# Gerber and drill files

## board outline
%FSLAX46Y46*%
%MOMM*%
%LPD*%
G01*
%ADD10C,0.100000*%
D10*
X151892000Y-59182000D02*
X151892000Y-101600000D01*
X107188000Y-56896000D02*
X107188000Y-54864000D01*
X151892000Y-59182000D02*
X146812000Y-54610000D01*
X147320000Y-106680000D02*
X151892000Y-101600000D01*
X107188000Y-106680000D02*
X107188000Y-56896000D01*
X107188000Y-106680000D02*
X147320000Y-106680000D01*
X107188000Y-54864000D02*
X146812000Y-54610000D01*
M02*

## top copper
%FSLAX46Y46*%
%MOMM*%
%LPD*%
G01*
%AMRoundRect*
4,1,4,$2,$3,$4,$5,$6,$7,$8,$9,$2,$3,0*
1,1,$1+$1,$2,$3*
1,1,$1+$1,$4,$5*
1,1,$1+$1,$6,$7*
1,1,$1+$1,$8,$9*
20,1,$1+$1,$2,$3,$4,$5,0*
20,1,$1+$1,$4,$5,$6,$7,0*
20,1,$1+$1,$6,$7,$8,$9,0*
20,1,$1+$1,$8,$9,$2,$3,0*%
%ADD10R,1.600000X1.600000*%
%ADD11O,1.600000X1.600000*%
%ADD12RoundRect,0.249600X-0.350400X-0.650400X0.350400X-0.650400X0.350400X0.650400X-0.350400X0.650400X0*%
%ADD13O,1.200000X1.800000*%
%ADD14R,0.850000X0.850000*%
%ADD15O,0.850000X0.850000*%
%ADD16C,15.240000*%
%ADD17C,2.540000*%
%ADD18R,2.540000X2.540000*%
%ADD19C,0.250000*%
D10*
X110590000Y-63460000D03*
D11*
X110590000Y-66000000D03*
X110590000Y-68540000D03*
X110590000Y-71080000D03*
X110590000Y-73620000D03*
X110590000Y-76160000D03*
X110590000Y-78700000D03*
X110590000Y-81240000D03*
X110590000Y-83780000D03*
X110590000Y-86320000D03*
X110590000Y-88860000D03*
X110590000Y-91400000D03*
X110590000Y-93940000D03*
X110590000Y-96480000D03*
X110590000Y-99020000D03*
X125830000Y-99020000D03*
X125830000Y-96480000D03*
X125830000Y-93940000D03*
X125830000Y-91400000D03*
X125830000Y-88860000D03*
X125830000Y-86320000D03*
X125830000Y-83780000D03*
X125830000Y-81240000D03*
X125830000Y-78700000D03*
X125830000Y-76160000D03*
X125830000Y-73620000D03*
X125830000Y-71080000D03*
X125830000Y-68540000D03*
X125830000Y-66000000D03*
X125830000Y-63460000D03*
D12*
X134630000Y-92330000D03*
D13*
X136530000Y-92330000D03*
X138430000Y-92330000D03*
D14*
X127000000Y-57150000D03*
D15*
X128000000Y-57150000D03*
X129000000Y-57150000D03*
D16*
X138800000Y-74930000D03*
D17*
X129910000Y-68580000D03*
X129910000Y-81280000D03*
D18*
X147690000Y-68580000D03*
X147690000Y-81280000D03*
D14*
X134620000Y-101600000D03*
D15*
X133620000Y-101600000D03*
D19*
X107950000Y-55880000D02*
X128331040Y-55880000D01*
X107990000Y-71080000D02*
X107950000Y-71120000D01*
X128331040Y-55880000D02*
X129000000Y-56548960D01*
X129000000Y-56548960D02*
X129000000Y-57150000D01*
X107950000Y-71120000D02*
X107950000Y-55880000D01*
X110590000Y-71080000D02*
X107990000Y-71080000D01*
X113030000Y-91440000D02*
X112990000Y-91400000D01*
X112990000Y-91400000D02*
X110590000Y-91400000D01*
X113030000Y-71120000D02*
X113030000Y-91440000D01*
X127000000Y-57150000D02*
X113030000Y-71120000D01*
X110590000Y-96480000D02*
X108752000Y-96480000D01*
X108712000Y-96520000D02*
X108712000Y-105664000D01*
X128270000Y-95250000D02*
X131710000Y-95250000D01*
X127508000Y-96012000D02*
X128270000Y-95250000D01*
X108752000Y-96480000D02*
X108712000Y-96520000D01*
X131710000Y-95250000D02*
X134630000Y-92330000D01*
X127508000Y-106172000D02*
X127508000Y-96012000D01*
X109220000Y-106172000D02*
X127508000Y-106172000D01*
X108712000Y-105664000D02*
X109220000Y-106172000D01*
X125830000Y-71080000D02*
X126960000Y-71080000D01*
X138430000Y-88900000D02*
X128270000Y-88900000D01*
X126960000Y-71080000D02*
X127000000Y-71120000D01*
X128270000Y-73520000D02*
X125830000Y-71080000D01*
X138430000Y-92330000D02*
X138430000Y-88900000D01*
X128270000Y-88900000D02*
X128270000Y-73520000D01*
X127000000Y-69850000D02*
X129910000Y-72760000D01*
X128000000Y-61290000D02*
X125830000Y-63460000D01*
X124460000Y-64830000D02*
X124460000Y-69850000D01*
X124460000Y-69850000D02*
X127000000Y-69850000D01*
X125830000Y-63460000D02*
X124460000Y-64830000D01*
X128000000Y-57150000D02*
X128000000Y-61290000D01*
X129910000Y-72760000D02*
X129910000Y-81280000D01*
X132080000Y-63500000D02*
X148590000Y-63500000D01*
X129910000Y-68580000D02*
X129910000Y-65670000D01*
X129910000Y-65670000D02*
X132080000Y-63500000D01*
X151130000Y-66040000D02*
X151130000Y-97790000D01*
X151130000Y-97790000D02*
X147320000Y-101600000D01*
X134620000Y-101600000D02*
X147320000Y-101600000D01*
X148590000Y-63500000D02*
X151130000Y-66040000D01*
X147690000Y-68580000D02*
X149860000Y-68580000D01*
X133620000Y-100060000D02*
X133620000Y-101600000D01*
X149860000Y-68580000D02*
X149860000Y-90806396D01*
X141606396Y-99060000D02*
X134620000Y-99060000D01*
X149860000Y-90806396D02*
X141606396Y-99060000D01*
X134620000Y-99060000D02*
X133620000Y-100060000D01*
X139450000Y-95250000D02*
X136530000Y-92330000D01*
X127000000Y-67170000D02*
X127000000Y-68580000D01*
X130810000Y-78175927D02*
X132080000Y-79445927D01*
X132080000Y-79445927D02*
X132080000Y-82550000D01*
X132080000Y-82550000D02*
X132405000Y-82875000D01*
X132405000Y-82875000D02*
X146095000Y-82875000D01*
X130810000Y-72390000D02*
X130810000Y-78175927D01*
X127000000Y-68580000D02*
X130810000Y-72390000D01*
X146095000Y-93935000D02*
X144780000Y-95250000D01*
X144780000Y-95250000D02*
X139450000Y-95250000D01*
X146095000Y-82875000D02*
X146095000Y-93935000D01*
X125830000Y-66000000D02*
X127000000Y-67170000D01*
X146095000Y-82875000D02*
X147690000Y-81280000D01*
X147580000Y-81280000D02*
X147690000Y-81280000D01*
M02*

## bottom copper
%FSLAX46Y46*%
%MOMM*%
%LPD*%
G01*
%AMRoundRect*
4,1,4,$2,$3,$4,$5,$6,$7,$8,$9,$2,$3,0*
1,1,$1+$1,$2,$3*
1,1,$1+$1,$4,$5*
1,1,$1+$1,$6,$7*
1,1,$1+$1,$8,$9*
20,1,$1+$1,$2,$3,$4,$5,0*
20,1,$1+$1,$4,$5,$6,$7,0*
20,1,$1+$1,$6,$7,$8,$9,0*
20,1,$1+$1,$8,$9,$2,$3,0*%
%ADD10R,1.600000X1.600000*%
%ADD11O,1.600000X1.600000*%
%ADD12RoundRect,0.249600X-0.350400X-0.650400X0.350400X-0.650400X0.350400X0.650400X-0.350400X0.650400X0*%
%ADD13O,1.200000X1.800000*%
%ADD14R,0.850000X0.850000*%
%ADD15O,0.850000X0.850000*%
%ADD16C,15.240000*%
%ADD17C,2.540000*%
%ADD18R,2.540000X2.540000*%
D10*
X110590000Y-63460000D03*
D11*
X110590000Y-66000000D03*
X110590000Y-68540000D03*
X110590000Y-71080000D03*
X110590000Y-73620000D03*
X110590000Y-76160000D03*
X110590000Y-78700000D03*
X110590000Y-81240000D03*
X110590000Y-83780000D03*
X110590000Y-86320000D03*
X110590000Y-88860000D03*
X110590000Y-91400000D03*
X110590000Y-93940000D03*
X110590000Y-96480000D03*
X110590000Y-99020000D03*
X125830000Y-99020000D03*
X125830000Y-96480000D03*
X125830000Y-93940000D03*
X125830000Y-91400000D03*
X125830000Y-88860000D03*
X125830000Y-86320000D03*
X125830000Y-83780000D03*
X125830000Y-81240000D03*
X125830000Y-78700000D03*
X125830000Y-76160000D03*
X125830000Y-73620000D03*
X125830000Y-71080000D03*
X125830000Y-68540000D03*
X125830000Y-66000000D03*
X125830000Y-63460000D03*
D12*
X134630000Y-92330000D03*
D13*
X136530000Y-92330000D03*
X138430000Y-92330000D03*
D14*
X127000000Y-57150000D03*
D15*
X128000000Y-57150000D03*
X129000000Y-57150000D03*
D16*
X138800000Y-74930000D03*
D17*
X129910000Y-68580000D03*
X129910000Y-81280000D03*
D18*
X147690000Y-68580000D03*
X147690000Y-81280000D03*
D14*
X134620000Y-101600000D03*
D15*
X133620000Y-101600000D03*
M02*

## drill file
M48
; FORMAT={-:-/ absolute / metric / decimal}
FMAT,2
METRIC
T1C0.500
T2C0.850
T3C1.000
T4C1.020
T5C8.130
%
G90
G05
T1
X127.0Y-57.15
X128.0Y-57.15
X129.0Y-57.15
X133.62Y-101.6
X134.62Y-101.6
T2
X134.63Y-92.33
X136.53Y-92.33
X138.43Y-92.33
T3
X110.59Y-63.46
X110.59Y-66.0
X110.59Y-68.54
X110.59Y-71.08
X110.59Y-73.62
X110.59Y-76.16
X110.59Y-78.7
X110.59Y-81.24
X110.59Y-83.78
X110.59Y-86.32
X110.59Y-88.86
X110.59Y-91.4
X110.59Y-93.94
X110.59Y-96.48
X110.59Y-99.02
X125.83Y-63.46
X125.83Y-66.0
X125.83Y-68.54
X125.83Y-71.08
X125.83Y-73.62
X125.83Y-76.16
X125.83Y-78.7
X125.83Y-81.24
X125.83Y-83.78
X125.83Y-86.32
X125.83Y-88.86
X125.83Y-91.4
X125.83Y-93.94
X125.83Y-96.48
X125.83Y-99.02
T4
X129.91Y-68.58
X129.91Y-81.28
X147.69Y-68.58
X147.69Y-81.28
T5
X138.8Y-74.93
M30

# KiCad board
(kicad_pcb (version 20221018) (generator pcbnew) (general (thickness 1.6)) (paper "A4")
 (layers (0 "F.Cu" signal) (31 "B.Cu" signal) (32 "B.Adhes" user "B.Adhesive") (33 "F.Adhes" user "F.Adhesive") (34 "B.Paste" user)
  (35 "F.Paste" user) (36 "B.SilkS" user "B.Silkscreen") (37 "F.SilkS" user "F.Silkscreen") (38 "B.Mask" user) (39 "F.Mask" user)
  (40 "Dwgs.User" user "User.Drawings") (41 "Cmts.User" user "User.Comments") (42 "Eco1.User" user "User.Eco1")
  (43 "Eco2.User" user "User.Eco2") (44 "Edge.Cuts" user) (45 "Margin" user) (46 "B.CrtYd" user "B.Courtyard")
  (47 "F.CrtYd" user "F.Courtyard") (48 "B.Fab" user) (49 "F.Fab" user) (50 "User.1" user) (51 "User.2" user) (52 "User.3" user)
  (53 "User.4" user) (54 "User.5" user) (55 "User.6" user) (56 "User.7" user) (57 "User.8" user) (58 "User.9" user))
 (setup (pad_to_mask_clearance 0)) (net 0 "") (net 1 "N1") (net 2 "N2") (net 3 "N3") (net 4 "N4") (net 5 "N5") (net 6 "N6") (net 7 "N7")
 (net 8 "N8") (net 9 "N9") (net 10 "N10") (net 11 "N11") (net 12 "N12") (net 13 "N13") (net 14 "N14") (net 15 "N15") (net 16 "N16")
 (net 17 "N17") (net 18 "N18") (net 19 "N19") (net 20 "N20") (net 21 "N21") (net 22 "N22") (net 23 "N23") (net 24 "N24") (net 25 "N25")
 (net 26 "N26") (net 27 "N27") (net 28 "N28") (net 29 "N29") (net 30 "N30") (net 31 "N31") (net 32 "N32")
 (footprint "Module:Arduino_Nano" (layer "F.Cu") (at 110.59 63.46)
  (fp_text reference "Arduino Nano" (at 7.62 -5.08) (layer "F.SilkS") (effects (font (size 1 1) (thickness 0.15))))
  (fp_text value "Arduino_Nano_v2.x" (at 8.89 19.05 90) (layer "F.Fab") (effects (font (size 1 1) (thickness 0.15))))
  (pad "1" thru_hole rect (at 0 0) (size 1.6 1.6) (drill 1) (layers "*.Cu" "*.Mask") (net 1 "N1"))
  (pad "2" thru_hole oval (at 0 2.54) (size 1.6 1.6) (drill 1) (layers "*.Cu" "*.Mask") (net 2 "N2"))
  (pad "3" thru_hole oval (at 0 5.08) (size 1.6 1.6) (drill 1) (layers "*.Cu" "*.Mask") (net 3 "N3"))
  (pad "4" thru_hole oval (at 0 7.62) (size 1.6 1.6) (drill 1) (layers "*.Cu" "*.Mask") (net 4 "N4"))
  (pad "5" thru_hole oval (at 0 10.16) (size 1.6 1.6) (drill 1) (layers "*.Cu" "*.Mask") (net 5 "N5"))
  (pad "6" thru_hole oval (at 0 12.7) (size 1.6 1.6) (drill 1) (layers "*.Cu" "*.Mask") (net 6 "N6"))
  (pad "7" thru_hole oval (at 0 15.24) (size 1.6 1.6) (drill 1) (layers "*.Cu" "*.Mask") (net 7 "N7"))
  (pad "8" thru_hole oval (at 0 17.78) (size 1.6 1.6) (drill 1) (layers "*.Cu" "*.Mask") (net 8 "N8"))
  (pad "9" thru_hole oval (at 0 20.32) (size 1.6 1.6) (drill 1) (layers "*.Cu" "*.Mask") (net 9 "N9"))
  (pad "10" thru_hole oval (at 0 22.86) (size 1.6 1.6) (drill 1) (layers "*.Cu" "*.Mask") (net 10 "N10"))
  (pad "11" thru_hole oval (at 0 25.4) (size 1.6 1.6) (drill 1) (layers "*.Cu" "*.Mask") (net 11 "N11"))
  (pad "12" thru_hole oval (at 0 27.94) (size 1.6 1.6) (drill 1) (layers "*.Cu" "*.Mask") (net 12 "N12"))
  (pad "13" thru_hole oval (at 0 30.48) (size 1.6 1.6) (drill 1) (layers "*.Cu" "*.Mask") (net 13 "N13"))
  (pad "14" thru_hole oval (at 0 33.02) (size 1.6 1.6) (drill 1) (layers "*.Cu" "*.Mask") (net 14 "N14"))
  (pad "15" thru_hole oval (at 0 35.56) (size 1.6 1.6) (drill 1) (layers "*.Cu" "*.Mask") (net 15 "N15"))
  (pad "16" thru_hole oval (at 15.24 35.56) (size 1.6 1.6) (drill 1) (layers "*.Cu" "*.Mask") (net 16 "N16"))
  (pad "17" thru_hole oval (at 15.24 33.02) (size 1.6 1.6) (drill 1) (layers "*.Cu" "*.Mask") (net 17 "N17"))
  (pad "18" thru_hole oval (at 15.24 30.48) (size 1.6 1.6) (drill 1) (layers "*.Cu" "*.Mask") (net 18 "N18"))
  (pad "19" thru_hole oval (at 15.24 27.94) (size 1.6 1.6) (drill 1) (layers "*.Cu" "*.Mask") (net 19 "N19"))
  (pad "20" thru_hole oval (at 15.24 25.4) (size 1.6 1.6) (drill 1) (layers "*.Cu" "*.Mask") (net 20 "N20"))
  (pad "21" thru_hole oval (at 15.24 22.86) (size 1.6 1.6) (drill 1) (layers "*.Cu" "*.Mask") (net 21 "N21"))
  (pad "22" thru_hole oval (at 15.24 20.32) (size 1.6 1.6) (drill 1) (layers "*.Cu" "*.Mask") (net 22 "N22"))
  (pad "23" thru_hole oval (at 15.24 17.78) (size 1.6 1.6) (drill 1) (layers "*.Cu" "*.Mask") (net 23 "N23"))
  (pad "24" thru_hole oval (at 15.24 15.24) (size 1.6 1.6) (drill 1) (layers "*.Cu" "*.Mask") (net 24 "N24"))
  (pad "25" thru_hole oval (at 15.24 12.7) (size 1.6 1.6) (drill 1) (layers "*.Cu" "*.Mask") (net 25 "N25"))
  (pad "26" thru_hole oval (at 15.24 10.16) (size 1.6 1.6) (drill 1) (layers "*.Cu" "*.Mask") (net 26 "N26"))
  (pad "27" thru_hole oval (at 15.24 7.62) (size 1.6 1.6) (drill 1) (layers "*.Cu" "*.Mask") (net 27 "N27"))
  (pad "28" thru_hole oval (at 15.24 5.08) (size 1.6 1.6) (drill 1) (layers "*.Cu" "*.Mask") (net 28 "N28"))
  (pad "29" thru_hole oval (at 15.24 2.54) (size 1.6 1.6) (drill 1) (layers "*.Cu" "*.Mask") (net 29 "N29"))
  (pad "30" thru_hole oval (at 15.24 0) (size 1.6 1.6) (drill 1) (layers "*.Cu" "*.Mask") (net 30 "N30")))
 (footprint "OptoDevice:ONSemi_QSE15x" (layer "F.Cu") (at 134.63 92.33)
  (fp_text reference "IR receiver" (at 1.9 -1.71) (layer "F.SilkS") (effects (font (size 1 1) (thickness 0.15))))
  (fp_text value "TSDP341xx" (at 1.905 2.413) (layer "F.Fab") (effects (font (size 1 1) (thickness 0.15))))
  (pad "1" thru_hole roundrect (at 0 0) (size 1.2 1.8) (drill 0.85) (layers "*.Cu" "*.Mask") (roundrect_rratio 0.208) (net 14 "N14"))
  (pad "2" thru_hole oval (at 1.9 0) (size 1.2 1.8) (drill 0.85) (layers "*.Cu" "*.Mask") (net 29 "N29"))
  (pad "3" thru_hole oval (at 3.8 0) (size 1.2 1.8) (drill 0.85) (layers "*.Cu" "*.Mask") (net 27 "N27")))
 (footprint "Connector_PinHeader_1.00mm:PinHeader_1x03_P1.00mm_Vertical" (layer "F.Cu") (at 127 57.15 90)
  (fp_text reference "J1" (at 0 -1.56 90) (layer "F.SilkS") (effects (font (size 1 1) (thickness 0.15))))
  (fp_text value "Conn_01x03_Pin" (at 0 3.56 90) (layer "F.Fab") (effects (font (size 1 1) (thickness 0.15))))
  (pad "1" thru_hole rect (at 0 0 90) (size 0.85 0.85) (drill 0.5) (layers "*.Cu" "*.Mask") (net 12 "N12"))
  (pad "2" thru_hole oval (at 0 1 90) (size 0.85 0.85) (drill 0.5) (layers "*.Cu" "*.Mask") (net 30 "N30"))
  (pad "3" thru_hole oval (at 0 2 90) (size 0.85 0.85) (drill 0.5) (layers "*.Cu" "*.Mask") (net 4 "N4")))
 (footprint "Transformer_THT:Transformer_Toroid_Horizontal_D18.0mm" (layer "F.Cu") (at 129.91 68.58)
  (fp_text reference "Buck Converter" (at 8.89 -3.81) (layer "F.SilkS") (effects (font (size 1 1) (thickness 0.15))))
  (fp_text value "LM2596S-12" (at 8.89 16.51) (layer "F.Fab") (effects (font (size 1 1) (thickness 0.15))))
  (pad "" thru_hole circle (at 8.89 6.35) (size 15.24 15.24) (drill 8.13) (layers "*.Cu" "*.Mask"))
  (pad "1" thru_hole circle (at 0 0) (size 2.54 2.54) (drill 1.02) (layers "*.Cu" "*.Mask") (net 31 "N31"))
  (pad "2" thru_hole circle (at 0 12.7) (size 2.54 2.54) (drill 1.02) (layers "*.Cu" "*.Mask") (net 30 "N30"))
  (pad "3" thru_hole rect (at 17.78 0) (size 2.54 2.54) (drill 1.02) (layers "*.Cu" "*.Mask") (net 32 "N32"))
  (pad "4" thru_hole rect (at 17.78 12.7) (size 2.54 2.54) (drill 1.02) (layers "*.Cu" "*.Mask") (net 29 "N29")))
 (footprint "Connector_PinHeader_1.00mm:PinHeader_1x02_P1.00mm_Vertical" (layer "F.Cu") (at 134.62 101.6 -90)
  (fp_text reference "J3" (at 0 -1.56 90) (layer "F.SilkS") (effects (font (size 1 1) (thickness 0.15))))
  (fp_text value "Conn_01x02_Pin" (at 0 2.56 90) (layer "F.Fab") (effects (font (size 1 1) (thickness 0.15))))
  (pad "1" thru_hole rect (at 0 0 270) (size 0.85 0.85) (drill 0.5) (layers "*.Cu" "*.Mask") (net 31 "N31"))
  (pad "2" thru_hole oval (at 0 1 270) (size 0.85 0.85) (drill 0.5) (layers "*.Cu" "*.Mask") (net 32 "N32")))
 (gr_line (start 151.892 59.182) (end 151.892 101.6) (stroke (width 0.1) (type default)) (layer "Edge.Cuts"))
 (gr_line (start 107.188 56.896) (end 107.188 54.864) (stroke (width 0.1) (type default)) (layer "Edge.Cuts"))
 (gr_line (start 151.892 59.182) (end 146.812 54.61) (stroke (width 0.1) (type default)) (layer "Edge.Cuts"))
 (gr_line (start 147.32 106.68) (end 151.892 101.6) (stroke (width 0.1) (type default)) (layer "Edge.Cuts"))
 (gr_line (start 107.188 106.68) (end 107.188 56.896) (stroke (width 0.1) (type default)) (layer "Edge.Cuts"))
 (gr_line (start 107.188 106.68) (end 147.32 106.68) (stroke (width 0.1) (type default)) (layer "Edge.Cuts"))
 (gr_line (start 107.188 54.864) (end 146.812 54.61) (stroke (width 0.1) (type default)) (layer "Edge.Cuts"))
 (segment (start 107.95 55.88) (end 128.33104 55.88) (width 0.25) (layer "F.Cu") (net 4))
 (segment (start 107.99 71.08) (end 107.95 71.12) (width 0.25) (layer "F.Cu") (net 4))
 (segment (start 128.33104 55.88) (end 129 56.54896) (width 0.25) (layer "F.Cu") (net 4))
 (segment (start 129 56.54896) (end 129 57.15) (width 0.25) (layer "F.Cu") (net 4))
 (segment (start 107.95 71.12) (end 107.95 55.88) (width 0.25) (layer "F.Cu") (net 4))
 (segment (start 110.59 71.08) (end 107.99 71.08) (width 0.25) (layer "F.Cu") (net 4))
 (segment (start 113.03 91.44) (end 112.99 91.4) (width 0.25) (layer "F.Cu") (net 12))
 (segment (start 112.99 91.4) (end 110.59 91.4) (width 0.25) (layer "F.Cu") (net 12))
 (segment (start 113.03 71.12) (end 113.03 91.44) (width 0.25) (layer "F.Cu") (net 12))
 (segment (start 127 57.15) (end 113.03 71.12) (width 0.25) (layer "F.Cu") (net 12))
 (segment (start 110.59 96.48) (end 108.752 96.48) (width 0.25) (layer "F.Cu") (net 14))
 (segment (start 108.712 96.52) (end 108.712 105.664) (width 0.25) (layer "F.Cu") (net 14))
 (segment (start 128.27 95.25) (end 131.71 95.25) (width 0.25) (layer "F.Cu") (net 14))
 (segment (start 127.508 96.012) (end 128.27 95.25) (width 0.25) (layer "F.Cu") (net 14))
 (segment (start 108.752 96.48) (end 108.712 96.52) (width 0.25) (layer "F.Cu") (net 14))
 (segment (start 131.71 95.25) (end 134.63 92.33) (width 0.25) (layer "F.Cu") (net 14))
 (segment (start 127.508 106.172) (end 127.508 96.012) (width 0.25) (layer "F.Cu") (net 14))
 (segment (start 109.22 106.172) (end 127.508 106.172) (width 0.25) (layer "F.Cu") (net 14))
 (segment (start 108.712 105.664) (end 109.22 106.172) (width 0.25) (layer "F.Cu") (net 14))
 (segment (start 125.83 71.08) (end 126.96 71.08) (width 0.25) (layer "F.Cu") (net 27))
 (segment (start 138.43 88.9) (end 128.27 88.9) (width 0.25) (layer "F.Cu") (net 27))
 (segment (start 126.96 71.08) (end 127 71.12) (width 0.25) (layer "F.Cu") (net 27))
 (segment (start 128.27 73.52) (end 125.83 71.08) (width 0.25) (layer "F.Cu") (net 27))
 (segment (start 138.43 92.33) (end 138.43 88.9) (width 0.25) (layer "F.Cu") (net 27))
 (segment (start 128.27 88.9) (end 128.27 73.52) (width 0.25) (layer "F.Cu") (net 27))
 (segment (start 127 69.85) (end 129.91 72.76) (width 0.25) (layer "F.Cu") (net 30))
 (segment (start 128 61.29) (end 125.83 63.46) (width 0.25) (layer "F.Cu") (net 30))
 (segment (start 124.46 64.83) (end 124.46 69.85) (width 0.25) (layer "F.Cu") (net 30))
 (segment (start 124.46 69.85) (end 127 69.85) (width 0.25) (layer "F.Cu") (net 30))
 (segment (start 125.83 63.46) (end 124.46 64.83) (width 0.25) (layer "F.Cu") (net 30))
 (segment (start 128 57.15) (end 128 61.29) (width 0.25) (layer "F.Cu") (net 30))
 (segment (start 129.91 72.76) (end 129.91 81.28) (width 0.25) (layer "F.Cu") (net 30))
 (segment (start 132.08 63.5) (end 148.59 63.5) (width 0.25) (layer "F.Cu") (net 31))
 (segment (start 129.91 68.58) (end 129.91 65.67) (width 0.25) (layer "F.Cu") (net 31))
 (segment (start 129.91 65.67) (end 132.08 63.5) (width 0.25) (layer "F.Cu") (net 31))
 (segment (start 151.13 66.04) (end 151.13 97.79) (width 0.25) (layer "F.Cu") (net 31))
 (segment (start 151.13 97.79) (end 147.32 101.6) (width 0.25) (layer "F.Cu") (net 31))
 (segment (start 134.62 101.6) (end 147.32 101.6) (width 0.25) (layer "F.Cu") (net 31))
 (segment (start 148.59 63.5) (end 151.13 66.04) (width 0.25) (layer "F.Cu") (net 31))
 (segment (start 147.69 68.58) (end 149.86 68.58) (width 0.25) (layer "F.Cu") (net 32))
 (segment (start 133.62 100.06) (end 133.62 101.6) (width 0.25) (layer "F.Cu") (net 32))
 (segment (start 149.86 68.58) (end 149.86 90.806396) (width 0.25) (layer "F.Cu") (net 32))
 (segment (start 141.606396 99.06) (end 134.62 99.06) (width 0.25) (layer "F.Cu") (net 32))
 (segment (start 149.86 90.806396) (end 141.606396 99.06) (width 0.25) (layer "F.Cu") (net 32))
 (segment (start 134.62 99.06) (end 133.62 100.06) (width 0.25) (layer "F.Cu") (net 32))
 (segment (start 139.45 95.25) (end 136.53 92.33) (width 0.25) (layer "F.Cu") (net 29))
 (segment (start 127 67.17) (end 127 68.58) (width 0.25) (layer "F.Cu") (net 29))
 (segment (start 130.81 78.175927) (end 132.08 79.445927) (width 0.25) (layer "F.Cu") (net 29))
 (segment (start 132.08 79.445927) (end 132.08 82.55) (width 0.25) (layer "F.Cu") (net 29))
 (segment (start 132.08 82.55) (end 132.405 82.875) (width 0.25) (layer "F.Cu") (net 29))
 (segment (start 132.405 82.875) (end 146.095 82.875) (width 0.25) (layer "F.Cu") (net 29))
 (segment (start 130.81 72.39) (end 130.81 78.175927) (width 0.25) (layer "F.Cu") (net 29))
 (segment (start 127 68.58) (end 130.81 72.39) (width 0.25) (layer "F.Cu") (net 29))
 (segment (start 146.095 93.935) (end 144.78 95.25) (width 0.25) (layer "F.Cu") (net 29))
 (segment (start 144.78 95.25) (end 139.45 95.25) (width 0.25) (layer "F.Cu") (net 29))
 (segment (start 146.095 82.875) (end 146.095 93.935) (width 0.25) (layer "F.Cu") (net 29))
 (segment (start 125.83 66) (end 127 67.17) (width 0.25) (layer "F.Cu") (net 29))
 (segment (start 146.095 82.875) (end 147.69 81.28) (width 0.25) (layer "F.Cu") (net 29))
 (segment (start 147.58 81.28) (end 147.69 81.28) (width 0.25) (layer "F.Cu") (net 29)))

